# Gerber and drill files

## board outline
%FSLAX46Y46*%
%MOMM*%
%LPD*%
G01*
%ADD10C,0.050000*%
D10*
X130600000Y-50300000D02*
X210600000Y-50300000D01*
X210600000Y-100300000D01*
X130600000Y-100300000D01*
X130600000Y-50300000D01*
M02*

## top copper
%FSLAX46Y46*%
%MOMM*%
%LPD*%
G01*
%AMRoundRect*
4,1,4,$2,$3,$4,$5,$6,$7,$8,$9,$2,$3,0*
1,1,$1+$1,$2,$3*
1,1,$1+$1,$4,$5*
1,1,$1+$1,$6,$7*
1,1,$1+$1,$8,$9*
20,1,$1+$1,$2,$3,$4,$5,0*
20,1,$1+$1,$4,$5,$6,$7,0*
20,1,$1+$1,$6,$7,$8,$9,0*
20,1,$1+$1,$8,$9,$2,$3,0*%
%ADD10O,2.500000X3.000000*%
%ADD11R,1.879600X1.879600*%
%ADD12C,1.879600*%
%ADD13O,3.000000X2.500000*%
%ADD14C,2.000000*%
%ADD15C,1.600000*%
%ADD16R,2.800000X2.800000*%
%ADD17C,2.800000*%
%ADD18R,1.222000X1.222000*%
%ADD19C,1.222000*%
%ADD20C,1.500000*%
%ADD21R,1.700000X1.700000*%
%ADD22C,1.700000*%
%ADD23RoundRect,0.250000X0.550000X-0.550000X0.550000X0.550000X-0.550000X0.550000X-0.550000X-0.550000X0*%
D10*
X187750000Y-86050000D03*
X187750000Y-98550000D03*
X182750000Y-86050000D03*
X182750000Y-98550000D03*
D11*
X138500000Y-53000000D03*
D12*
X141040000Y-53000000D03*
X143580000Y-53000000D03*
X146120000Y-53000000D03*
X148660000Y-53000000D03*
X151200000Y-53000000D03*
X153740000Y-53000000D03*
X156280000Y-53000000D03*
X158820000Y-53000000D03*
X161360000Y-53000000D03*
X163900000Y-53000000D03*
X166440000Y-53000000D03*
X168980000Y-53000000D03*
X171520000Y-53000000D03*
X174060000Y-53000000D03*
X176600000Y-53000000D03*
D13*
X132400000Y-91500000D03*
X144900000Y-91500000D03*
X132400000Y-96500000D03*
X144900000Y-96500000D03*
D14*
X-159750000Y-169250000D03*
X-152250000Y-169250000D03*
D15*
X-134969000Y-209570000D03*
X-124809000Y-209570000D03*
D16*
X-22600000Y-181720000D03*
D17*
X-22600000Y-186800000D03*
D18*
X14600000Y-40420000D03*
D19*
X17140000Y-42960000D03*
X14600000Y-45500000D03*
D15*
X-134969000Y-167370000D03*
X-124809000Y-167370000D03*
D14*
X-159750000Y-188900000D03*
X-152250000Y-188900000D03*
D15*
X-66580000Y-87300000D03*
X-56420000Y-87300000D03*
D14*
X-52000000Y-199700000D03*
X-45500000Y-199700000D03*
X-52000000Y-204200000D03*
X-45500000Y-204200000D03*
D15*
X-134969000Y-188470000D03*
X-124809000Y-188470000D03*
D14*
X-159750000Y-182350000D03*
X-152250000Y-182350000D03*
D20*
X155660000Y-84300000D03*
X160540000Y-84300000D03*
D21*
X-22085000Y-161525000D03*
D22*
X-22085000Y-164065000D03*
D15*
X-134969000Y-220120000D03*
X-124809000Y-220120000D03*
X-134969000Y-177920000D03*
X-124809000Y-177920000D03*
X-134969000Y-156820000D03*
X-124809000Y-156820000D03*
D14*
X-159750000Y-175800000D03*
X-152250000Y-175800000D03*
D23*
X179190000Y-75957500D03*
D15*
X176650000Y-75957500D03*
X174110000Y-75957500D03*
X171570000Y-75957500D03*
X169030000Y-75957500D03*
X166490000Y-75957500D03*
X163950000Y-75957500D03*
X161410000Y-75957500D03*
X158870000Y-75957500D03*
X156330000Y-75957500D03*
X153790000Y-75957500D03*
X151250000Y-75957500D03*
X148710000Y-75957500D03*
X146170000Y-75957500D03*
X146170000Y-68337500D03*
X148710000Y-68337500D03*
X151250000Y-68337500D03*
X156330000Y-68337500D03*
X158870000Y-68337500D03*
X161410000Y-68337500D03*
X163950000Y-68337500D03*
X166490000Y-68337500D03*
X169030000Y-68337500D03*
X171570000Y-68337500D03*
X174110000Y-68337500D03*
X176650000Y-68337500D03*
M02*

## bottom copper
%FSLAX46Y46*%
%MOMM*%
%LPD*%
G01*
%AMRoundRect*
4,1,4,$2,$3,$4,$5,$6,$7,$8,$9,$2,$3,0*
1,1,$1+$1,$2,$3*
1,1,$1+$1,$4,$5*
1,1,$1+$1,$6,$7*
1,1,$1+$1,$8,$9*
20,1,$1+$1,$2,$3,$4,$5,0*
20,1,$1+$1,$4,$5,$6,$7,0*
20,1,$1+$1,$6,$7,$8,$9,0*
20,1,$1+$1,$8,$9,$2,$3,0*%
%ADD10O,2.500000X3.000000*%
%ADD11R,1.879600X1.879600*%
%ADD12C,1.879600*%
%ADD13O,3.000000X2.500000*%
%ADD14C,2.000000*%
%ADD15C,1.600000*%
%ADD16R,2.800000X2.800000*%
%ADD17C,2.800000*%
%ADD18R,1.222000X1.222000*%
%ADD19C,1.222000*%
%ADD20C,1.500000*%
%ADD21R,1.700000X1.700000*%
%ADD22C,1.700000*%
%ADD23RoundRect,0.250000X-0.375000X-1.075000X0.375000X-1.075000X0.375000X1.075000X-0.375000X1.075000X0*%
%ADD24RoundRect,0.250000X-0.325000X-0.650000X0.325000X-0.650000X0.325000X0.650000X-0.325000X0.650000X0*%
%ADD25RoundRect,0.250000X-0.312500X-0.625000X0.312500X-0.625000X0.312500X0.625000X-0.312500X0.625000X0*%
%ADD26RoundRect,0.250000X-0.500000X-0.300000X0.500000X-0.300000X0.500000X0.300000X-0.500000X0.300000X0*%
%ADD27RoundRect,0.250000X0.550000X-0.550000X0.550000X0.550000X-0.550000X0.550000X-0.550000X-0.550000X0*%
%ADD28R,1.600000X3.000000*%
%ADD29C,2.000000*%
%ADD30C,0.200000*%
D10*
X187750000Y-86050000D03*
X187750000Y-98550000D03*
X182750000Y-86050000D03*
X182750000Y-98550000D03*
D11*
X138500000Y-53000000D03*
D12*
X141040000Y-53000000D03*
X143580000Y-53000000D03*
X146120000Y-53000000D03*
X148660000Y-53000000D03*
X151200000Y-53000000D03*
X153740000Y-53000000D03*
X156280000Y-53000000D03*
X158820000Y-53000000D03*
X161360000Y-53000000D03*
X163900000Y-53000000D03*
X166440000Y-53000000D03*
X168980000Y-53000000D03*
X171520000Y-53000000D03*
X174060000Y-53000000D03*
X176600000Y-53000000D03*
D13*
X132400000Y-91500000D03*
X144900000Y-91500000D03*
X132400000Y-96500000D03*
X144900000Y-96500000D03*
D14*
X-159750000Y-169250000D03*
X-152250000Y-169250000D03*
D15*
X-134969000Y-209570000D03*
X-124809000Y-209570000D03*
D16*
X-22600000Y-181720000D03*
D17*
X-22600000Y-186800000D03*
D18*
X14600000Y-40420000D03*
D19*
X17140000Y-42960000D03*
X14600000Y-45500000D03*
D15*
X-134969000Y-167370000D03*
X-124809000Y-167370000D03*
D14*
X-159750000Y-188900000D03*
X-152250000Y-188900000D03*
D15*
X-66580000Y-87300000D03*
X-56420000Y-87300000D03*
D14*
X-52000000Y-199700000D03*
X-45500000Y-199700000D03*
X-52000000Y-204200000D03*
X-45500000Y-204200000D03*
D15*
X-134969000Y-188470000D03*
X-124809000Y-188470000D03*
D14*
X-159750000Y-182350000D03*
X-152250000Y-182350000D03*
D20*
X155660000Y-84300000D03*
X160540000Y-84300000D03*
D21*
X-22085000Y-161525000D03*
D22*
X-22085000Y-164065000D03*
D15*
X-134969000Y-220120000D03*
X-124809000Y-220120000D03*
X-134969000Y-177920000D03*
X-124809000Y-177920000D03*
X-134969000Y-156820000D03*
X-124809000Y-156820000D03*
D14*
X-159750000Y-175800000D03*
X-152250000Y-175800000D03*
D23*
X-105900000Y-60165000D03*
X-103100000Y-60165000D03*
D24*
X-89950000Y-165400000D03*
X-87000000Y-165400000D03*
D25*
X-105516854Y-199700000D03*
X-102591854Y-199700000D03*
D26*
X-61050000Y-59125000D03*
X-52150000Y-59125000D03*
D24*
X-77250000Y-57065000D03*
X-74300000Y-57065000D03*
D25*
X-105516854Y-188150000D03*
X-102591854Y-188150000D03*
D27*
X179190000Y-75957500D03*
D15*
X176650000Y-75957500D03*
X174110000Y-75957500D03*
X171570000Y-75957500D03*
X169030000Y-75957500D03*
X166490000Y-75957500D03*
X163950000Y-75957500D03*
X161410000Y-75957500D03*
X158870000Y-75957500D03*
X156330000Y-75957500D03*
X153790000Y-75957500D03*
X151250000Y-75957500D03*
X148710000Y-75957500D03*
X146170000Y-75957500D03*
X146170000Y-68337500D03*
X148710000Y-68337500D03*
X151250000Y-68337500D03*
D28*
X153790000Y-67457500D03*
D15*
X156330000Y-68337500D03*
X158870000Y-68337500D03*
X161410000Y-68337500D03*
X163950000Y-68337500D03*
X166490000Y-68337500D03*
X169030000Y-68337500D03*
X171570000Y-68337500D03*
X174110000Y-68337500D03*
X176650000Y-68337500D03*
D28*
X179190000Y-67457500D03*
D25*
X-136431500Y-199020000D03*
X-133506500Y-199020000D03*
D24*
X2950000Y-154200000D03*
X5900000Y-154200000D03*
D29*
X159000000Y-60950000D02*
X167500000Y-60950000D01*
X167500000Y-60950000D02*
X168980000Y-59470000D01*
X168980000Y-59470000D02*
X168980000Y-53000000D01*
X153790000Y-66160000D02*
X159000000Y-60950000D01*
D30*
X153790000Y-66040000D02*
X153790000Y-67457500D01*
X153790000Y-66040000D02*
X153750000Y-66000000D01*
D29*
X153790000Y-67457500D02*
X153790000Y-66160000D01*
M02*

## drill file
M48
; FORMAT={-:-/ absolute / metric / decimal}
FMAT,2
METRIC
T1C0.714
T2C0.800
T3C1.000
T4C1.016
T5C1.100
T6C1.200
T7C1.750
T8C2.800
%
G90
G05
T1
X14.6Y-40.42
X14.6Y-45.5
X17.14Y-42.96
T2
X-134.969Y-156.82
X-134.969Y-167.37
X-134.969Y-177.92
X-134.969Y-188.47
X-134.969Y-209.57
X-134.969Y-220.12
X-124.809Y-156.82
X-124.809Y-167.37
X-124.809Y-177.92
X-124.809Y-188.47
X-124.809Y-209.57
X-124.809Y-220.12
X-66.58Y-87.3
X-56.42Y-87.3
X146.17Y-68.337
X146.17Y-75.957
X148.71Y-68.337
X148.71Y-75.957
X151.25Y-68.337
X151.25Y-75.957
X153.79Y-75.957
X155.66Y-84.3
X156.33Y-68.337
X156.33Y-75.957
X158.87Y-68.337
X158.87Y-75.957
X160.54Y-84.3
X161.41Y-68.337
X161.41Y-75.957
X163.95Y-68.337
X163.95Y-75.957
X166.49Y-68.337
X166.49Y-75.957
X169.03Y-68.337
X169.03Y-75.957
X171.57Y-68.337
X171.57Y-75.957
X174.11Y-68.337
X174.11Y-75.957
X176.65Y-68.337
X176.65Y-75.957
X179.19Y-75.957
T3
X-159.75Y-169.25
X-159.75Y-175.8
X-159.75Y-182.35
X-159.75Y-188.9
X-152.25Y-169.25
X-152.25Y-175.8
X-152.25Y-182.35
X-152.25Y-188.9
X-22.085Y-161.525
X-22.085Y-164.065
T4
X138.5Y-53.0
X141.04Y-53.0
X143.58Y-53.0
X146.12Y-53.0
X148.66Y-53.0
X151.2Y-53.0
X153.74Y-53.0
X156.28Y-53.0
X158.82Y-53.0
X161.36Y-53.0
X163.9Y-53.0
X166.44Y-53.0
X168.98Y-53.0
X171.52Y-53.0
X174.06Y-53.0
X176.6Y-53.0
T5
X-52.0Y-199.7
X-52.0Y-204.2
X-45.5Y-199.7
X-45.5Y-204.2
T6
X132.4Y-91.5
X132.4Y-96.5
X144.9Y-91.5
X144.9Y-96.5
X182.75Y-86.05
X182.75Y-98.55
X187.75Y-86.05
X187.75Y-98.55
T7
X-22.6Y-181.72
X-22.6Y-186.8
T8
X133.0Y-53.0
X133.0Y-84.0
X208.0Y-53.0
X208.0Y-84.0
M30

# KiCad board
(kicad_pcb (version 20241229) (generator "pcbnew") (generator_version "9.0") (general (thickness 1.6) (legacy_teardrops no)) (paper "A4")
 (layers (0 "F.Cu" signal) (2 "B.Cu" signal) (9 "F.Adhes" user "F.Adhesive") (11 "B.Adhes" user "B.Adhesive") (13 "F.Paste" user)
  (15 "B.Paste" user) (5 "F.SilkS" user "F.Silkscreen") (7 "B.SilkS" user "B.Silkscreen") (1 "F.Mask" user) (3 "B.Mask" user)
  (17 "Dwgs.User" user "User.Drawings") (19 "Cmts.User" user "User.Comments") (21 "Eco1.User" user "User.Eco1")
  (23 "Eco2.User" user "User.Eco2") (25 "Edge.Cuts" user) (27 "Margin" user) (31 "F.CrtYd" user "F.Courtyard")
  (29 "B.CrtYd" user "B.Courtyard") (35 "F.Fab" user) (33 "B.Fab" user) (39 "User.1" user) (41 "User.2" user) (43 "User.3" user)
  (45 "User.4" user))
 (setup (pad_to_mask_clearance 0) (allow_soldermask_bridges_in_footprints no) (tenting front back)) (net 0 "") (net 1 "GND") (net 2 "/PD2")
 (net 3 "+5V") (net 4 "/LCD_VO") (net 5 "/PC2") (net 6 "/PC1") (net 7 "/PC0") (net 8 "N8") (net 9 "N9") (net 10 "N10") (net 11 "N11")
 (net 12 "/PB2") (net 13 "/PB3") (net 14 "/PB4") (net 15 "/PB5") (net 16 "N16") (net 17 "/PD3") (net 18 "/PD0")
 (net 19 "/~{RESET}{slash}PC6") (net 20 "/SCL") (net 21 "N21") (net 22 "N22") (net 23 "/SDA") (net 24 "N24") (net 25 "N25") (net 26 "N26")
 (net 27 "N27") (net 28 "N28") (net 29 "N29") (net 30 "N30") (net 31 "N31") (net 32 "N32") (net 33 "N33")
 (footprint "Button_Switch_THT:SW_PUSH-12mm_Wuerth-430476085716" (layer "F.Cu") (at 187.75 86.05 -90)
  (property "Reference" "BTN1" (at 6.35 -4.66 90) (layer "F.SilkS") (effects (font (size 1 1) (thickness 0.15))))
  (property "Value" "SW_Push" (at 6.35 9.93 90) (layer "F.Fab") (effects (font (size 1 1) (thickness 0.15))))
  (pad "1" thru_hole oval (at 0 0 270) (size 3 2.5) (drill 1.2) (layers "*.Cu" "*.Mask") (remove_unused_layers no) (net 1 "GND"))
  (pad "1" thru_hole oval (at 12.5 0 270) (size 3 2.5) (drill 1.2) (layers "*.Cu" "*.Mask") (remove_unused_layers no) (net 1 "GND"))
  (pad "2" thru_hole oval (at 0 5 270) (size 3 2.5) (drill 1.2) (layers "*.Cu" "*.Mask") (remove_unused_layers no) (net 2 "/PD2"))
  (pad "2" thru_hole oval (at 12.5 5 270) (size 3 2.5) (drill 1.2) (layers "*.Cu" "*.Mask") (remove_unused_layers no) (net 2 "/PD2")))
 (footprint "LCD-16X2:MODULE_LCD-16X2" (layer "F.Cu") (at 170.5 68.5)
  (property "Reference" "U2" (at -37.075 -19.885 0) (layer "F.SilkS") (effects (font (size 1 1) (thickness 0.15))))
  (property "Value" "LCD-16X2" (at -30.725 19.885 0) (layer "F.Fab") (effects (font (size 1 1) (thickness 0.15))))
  (pad "" np_thru_hole circle (at -37.5 -15.5) (size 2.8 2.8) (drill 2.8) (layers "*.Cu" "*.Mask"))
  (pad "" np_thru_hole circle (at -37.5 15.5) (size 2.8 2.8) (drill 2.8) (layers "*.Cu" "*.Mask"))
  (pad "" np_thru_hole circle (at 37.5 -15.5) (size 2.8 2.8) (drill 2.8) (layers "*.Cu" "*.Mask"))
  (pad "" np_thru_hole circle (at 37.5 15.5) (size 2.8 2.8) (drill 2.8) (layers "*.Cu" "*.Mask"))
  (pad "1" thru_hole rect (at -32 -15.5) (size 1.8796 1.8796) (drill 1.016) (layers "*.Cu" "*.Mask") (remove_unused_layers no) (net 1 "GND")
   (solder_mask_margin 0.102))
  (pad "2" thru_hole circle (at -29.46 -15.5) (size 1.8796 1.8796) (drill 1.016) (layers "*.Cu" "*.Mask") (remove_unused_layers no)
   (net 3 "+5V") (solder_mask_margin 0.102))
  (pad "3" thru_hole circle (at -26.92 -15.5) (size 1.8796 1.8796) (drill 1.016) (layers "*.Cu" "*.Mask") (remove_unused_layers no)
   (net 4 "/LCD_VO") (solder_mask_margin 0.102))
  (pad "4" thru_hole circle (at -24.38 -15.5) (size 1.8796 1.8796) (drill 1.016) (layers "*.Cu" "*.Mask") (remove_unused_layers no)
   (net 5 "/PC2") (solder_mask_margin 0.102))
  (pad "5" thru_hole circle (at -21.84 -15.5) (size 1.8796 1.8796) (drill 1.016) (layers "*.Cu" "*.Mask") (remove_unused_layers no)
   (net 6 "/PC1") (solder_mask_margin 0.102))
  (pad "6" thru_hole circle (at -19.3 -15.5) (size 1.8796 1.8796) (drill 1.016) (layers "*.Cu" "*.Mask") (remove_unused_layers no)
   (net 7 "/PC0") (solder_mask_margin 0.102))
  (pad "7" thru_hole circle (at -16.76 -15.5) (size 1.8796 1.8796) (drill 1.016) (layers "*.Cu" "*.Mask") (remove_unused_layers no)
   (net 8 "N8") (solder_mask_margin 0.102))
  (pad "8" thru_hole circle (at -14.22 -15.5) (size 1.8796 1.8796) (drill 1.016) (layers "*.Cu" "*.Mask") (remove_unused_layers no)
   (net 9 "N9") (solder_mask_margin 0.102))
  (pad "9" thru_hole circle (at -11.68 -15.5) (size 1.8796 1.8796) (drill 1.016) (layers "*.Cu" "*.Mask") (remove_unused_layers no)
   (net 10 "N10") (solder_mask_margin 0.102))
  (pad "10" thru_hole circle (at -9.14 -15.5) (size 1.8796 1.8796) (drill 1.016) (layers "*.Cu" "*.Mask") (remove_unused_layers no)
   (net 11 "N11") (solder_mask_margin 0.102))
  (pad "11" thru_hole circle (at -6.6 -15.5) (size 1.8796 1.8796) (drill 1.016) (layers "*.Cu" "*.Mask") (remove_unused_layers no)
   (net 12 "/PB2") (solder_mask_margin 0.102))
  (pad "12" thru_hole circle (at -4.06 -15.5) (size 1.8796 1.8796) (drill 1.016) (layers "*.Cu" "*.Mask") (remove_unused_layers no)
   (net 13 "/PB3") (solder_mask_margin 0.102))
  (pad "13" thru_hole circle (at -1.52 -15.5) (size 1.8796 1.8796) (drill 1.016) (layers "*.Cu" "*.Mask") (remove_unused_layers no)
   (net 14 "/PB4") (solder_mask_margin 0.102))
  (pad "14" thru_hole circle (at 1.02 -15.5) (size 1.8796 1.8796) (drill 1.016) (layers "*.Cu" "*.Mask") (remove_unused_layers no)
   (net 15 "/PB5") (solder_mask_margin 0.102))
  (pad "15" thru_hole circle (at 3.56 -15.5) (size 1.8796 1.8796) (drill 1.016) (layers "*.Cu" "*.Mask") (remove_unused_layers no)
   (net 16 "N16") (solder_mask_margin 0.102))
  (pad "16" thru_hole circle (at 6.1 -15.5) (size 1.8796 1.8796) (drill 1.016) (layers "*.Cu" "*.Mask") (remove_unused_layers no)
   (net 1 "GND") (solder_mask_margin 0.102)))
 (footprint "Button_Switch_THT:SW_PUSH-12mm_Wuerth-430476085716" (layer "F.Cu") (at 132.4 91.5)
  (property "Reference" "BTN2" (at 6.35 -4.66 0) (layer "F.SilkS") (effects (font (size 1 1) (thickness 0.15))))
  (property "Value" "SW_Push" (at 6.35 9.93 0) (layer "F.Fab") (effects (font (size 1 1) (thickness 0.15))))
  (pad "1" thru_hole oval (at 0 0) (size 3 2.5) (drill 1.2) (layers "*.Cu" "*.Mask") (remove_unused_layers no) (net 1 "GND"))
  (pad "1" thru_hole oval (at 12.5 0) (size 3 2.5) (drill 1.2) (layers "*.Cu" "*.Mask") (remove_unused_layers no) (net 1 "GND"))
  (pad "2" thru_hole oval (at 0 5) (size 3 2.5) (drill 1.2) (layers "*.Cu" "*.Mask") (remove_unused_layers no) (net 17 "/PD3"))
  (pad "2" thru_hole oval (at 12.5 5) (size 3 2.5) (drill 1.2) (layers "*.Cu" "*.Mask") (remove_unused_layers no) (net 17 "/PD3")))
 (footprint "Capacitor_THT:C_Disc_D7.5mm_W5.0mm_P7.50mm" (layer "F.Cu") (at -159.75 169.25)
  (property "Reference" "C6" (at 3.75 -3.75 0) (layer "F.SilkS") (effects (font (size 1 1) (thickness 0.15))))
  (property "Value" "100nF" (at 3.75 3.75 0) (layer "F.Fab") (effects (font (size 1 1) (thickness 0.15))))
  (pad "1" thru_hole circle (at 0 0) (size 2 2) (drill 1) (layers "*.Cu" "*.Mask") (remove_unused_layers no) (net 1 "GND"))
  (pad "2" thru_hole circle (at 7.5 0) (size 2 2) (drill 1) (layers "*.Cu" "*.Mask") (remove_unused_layers no) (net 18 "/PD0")))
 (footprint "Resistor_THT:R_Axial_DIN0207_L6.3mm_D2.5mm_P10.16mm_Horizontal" (layer "F.Cu") (at -134.969 209.57)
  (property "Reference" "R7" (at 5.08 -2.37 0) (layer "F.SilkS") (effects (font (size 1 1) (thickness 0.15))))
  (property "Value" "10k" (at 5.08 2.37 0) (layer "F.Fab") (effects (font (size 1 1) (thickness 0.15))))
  (pad "1" thru_hole circle (at 0 0) (size 1.6 1.6) (drill 0.8) (layers "*.Cu" "*.Mask") (remove_unused_layers no) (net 3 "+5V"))
  (pad "2" thru_hole circle (at 10.16 0) (size 1.6 1.6) (drill 0.8) (layers "*.Cu" "*.Mask") (remove_unused_layers no)
   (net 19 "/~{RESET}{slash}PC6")))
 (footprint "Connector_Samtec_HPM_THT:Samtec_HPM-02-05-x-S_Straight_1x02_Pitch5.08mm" (layer "F.Cu") (at -22.6 181.72)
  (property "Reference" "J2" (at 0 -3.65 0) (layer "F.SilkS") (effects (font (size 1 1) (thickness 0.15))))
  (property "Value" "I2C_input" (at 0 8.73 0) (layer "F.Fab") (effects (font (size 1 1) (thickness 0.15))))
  (pad "1" thru_hole rect (at 0 0) (size 2.8 2.8) (drill 1.75) (layers "*.Cu" "*.Mask") (remove_unused_layers no) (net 3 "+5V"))
  (pad "2" thru_hole circle (at 0 5.08) (size 2.8 2.8) (drill 1.75) (layers "*.Cu" "*.Mask") (remove_unused_layers no) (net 1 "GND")))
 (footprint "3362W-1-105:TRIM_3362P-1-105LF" (layer "F.Cu") (at 14.6 42.96 -90)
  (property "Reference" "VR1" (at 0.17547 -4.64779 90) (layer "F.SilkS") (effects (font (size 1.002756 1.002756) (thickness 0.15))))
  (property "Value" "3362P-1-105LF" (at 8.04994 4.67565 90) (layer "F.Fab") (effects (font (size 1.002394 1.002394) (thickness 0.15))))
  (pad "1" thru_hole rect (at -2.54 0 270) (size 1.222 1.222) (drill 0.714) (layers "*.Cu" "*.Mask") (remove_unused_layers no) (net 3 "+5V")
   (solder_mask_margin 0.102))
  (pad "2" thru_hole circle (at 0 -2.54 270) (size 1.222 1.222) (drill 0.714) (layers "*.Cu" "*.Mask") (remove_unused_layers no)
   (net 4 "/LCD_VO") (solder_mask_margin 0.102))
  (pad "3" thru_hole circle (at 2.54 0 270) (size 1.222 1.222) (drill 0.714) (layers "*.Cu" "*.Mask") (remove_unused_layers no)
   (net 1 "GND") (solder_mask_margin 0.102)))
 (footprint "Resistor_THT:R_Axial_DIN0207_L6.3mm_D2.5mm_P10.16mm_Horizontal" (layer "F.Cu") (at -134.969 167.37)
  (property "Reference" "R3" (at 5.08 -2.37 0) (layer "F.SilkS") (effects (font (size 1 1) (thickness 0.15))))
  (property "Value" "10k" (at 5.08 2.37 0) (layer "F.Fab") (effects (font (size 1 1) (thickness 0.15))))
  (pad "1" thru_hole circle (at 0 0) (size 1.6 1.6) (drill 0.8) (layers "*.Cu" "*.Mask") (remove_unused_layers no) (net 3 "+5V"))
  (pad "2" thru_hole circle (at 10.16 0) (size 1.6 1.6) (drill 0.8) (layers "*.Cu" "*.Mask") (remove_unused_layers no) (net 17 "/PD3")))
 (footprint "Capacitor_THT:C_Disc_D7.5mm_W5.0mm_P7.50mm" (layer "F.Cu") (at -159.75 188.9)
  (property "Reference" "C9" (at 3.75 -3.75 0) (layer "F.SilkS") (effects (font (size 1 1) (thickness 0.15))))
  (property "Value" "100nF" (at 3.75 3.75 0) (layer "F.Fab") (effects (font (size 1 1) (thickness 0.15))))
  (pad "1" thru_hole circle (at 0 0) (size 2 2) (drill 1) (layers "*.Cu" "*.Mask") (remove_unused_layers no) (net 1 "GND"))
  (pad "2" thru_hole circle (at 7.5 0) (size 2 2) (drill 1) (layers "*.Cu" "*.Mask") (remove_unused_layers no) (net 17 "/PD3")))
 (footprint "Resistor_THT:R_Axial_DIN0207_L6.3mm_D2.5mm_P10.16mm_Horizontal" (layer "F.Cu") (at -66.58 87.3)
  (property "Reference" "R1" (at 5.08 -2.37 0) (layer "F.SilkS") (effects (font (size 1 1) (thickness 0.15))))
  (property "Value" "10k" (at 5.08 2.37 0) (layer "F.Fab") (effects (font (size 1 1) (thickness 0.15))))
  (pad "1" thru_hole circle (at 0 0) (size 1.6 1.6) (drill 0.8) (layers "*.Cu" "*.Mask") (remove_unused_layers no) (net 3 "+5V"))
  (pad "2" thru_hole circle (at 10.16 0) (size 1.6 1.6) (drill 0.8) (layers "*.Cu" "*.Mask") (remove_unused_layers no) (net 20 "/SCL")))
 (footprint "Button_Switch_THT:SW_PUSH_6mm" (layer "F.Cu") (at -52 199.7)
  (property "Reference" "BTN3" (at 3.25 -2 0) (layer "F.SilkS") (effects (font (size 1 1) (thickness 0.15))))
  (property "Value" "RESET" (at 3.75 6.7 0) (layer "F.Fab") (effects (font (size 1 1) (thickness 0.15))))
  (pad "1" thru_hole circle (at 0 0 90) (size 2 2) (drill 1.1) (layers "*.Cu" "*.Mask") (remove_unused_layers no) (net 1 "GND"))
  (pad "1" thru_hole circle (at 6.5 0 90) (size 2 2) (drill 1.1) (layers "*.Cu" "*.Mask") (remove_unused_layers no) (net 1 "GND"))
  (pad "2" thru_hole circle (at 0 4.5 90) (size 2 2) (drill 1.1) (layers "*.Cu" "*.Mask") (remove_unused_layers no)
   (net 19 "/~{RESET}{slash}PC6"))
  (pad "2" thru_hole circle (at 6.5 4.5 90) (size 2 2) (drill 1.1) (layers "*.Cu" "*.Mask") (remove_unused_layers no)
   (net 19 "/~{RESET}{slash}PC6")))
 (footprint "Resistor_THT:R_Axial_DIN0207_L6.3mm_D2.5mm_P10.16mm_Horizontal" (layer "F.Cu") (at -134.969 188.47)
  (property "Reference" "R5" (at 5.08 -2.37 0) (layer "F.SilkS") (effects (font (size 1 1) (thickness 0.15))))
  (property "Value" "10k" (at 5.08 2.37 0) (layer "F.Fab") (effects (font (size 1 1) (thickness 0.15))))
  (pad "1" thru_hole circle (at 0 0) (size 1.6 1.6) (drill 0.8) (layers "*.Cu" "*.Mask") (remove_unused_layers no) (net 3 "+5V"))
  (pad "2" thru_hole circle (at 10.16 0) (size 1.6 1.6) (drill 0.8) (layers "*.Cu" "*.Mask") (remove_unused_layers no) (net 18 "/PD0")))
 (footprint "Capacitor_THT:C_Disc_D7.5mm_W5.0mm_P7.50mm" (layer "F.Cu") (at -159.75 182.35)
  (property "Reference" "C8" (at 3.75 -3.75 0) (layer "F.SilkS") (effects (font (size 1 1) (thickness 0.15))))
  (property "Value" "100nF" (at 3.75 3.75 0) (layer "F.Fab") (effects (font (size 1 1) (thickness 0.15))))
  (pad "1" thru_hole circle (at 0 0) (size 2 2) (drill 1) (layers "*.Cu" "*.Mask") (remove_unused_layers no) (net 1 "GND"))
  (pad "2" thru_hole circle (at 7.5 0) (size 2 2) (drill 1) (layers "*.Cu" "*.Mask") (remove_unused_layers no) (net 2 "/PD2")))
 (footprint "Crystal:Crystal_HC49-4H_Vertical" (layer "F.Cu") (at 155.66 84.3)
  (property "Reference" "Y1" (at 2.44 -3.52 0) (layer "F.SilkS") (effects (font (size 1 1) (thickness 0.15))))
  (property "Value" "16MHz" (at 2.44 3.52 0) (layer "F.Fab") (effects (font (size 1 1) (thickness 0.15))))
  (pad "1" thru_hole circle (at 0 0) (size 1.5 1.5) (drill 0.8) (layers "*.Cu" "*.Mask") (remove_unused_layers no) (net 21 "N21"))
  (pad "2" thru_hole circle (at 4.88 0) (size 1.5 1.5) (drill 0.8) (layers "*.Cu" "*.Mask") (remove_unused_layers no) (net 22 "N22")))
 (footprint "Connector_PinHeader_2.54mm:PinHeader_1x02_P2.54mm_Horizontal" (layer "F.Cu") (at -22.085 161.525)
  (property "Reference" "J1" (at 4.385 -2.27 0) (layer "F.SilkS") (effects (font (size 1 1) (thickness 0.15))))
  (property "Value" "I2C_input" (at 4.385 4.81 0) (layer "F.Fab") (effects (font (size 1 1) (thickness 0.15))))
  (pad "1" thru_hole rect (at 0 0) (size 1.7 1.7) (drill 1) (layers "*.Cu" "*.Mask") (remove_unused_layers no) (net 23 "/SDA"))
  (pad "2" thru_hole circle (at 0 2.54) (size 1.7 1.7) (drill 1) (layers "*.Cu" "*.Mask") (remove_unused_layers no) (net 20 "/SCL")))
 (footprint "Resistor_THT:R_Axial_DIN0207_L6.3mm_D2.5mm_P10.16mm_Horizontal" (layer "F.Cu") (at -134.969 220.12)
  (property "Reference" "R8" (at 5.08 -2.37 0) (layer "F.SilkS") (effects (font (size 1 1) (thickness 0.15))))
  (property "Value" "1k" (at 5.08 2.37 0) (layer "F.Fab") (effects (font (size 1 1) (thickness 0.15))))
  (pad "1" thru_hole circle (at 0 0) (size 1.6 1.6) (drill 0.8) (layers "*.Cu" "*.Mask") (remove_unused_layers no) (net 3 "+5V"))
  (pad "2" thru_hole circle (at 10.16 0) (size 1.6 1.6) (drill 0.8) (layers "*.Cu" "*.Mask") (remove_unused_layers no) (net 16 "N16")))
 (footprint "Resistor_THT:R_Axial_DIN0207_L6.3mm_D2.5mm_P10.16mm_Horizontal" (layer "F.Cu") (at -134.969 177.92)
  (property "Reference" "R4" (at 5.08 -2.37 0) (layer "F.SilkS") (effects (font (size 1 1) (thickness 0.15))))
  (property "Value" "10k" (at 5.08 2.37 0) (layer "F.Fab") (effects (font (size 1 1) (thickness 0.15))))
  (pad "1" thru_hole circle (at 0 0) (size 1.6 1.6) (drill 0.8) (layers "*.Cu" "*.Mask") (remove_unused_layers no) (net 3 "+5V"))
  (pad "2" thru_hole circle (at 10.16 0) (size 1.6 1.6) (drill 0.8) (layers "*.Cu" "*.Mask") (remove_unused_layers no) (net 2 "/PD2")))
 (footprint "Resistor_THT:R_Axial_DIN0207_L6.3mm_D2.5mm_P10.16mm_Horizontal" (layer "F.Cu") (at -134.969 156.82)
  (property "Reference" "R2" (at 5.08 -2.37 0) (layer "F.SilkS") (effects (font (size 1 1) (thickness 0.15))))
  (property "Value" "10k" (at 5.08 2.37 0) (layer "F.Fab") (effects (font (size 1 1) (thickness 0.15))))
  (pad "1" thru_hole circle (at 0 0) (size 1.6 1.6) (drill 0.8) (layers "*.Cu" "*.Mask") (remove_unused_layers no) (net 3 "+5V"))
  (pad "2" thru_hole circle (at 10.16 0) (size 1.6 1.6) (drill 0.8) (layers "*.Cu" "*.Mask") (remove_unused_layers no) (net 23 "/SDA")))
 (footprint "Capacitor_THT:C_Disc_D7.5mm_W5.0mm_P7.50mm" (layer "F.Cu") (at -159.75 175.8)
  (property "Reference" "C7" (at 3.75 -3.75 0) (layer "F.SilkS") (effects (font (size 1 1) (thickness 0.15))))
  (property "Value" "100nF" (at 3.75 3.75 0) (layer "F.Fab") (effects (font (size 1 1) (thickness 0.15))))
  (pad "1" thru_hole circle (at 0 0) (size 2 2) (drill 1) (layers "*.Cu" "*.Mask") (remove_unused_layers no) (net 1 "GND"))
  (pad "2" thru_hole circle (at 7.5 0) (size 2 2) (drill 1) (layers "*.Cu" "*.Mask") (remove_unused_layers no)
   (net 19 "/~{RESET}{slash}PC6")))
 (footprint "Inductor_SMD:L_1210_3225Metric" (layer "B.Cu") (at -104.5 60.165)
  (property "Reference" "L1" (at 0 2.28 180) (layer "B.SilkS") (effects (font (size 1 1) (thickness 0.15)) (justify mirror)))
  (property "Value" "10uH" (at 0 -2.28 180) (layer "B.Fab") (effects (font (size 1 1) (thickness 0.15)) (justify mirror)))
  (pad "1" smd roundrect (at -1.4 0) (size 1.25 2.65) (layers "B.Cu" "B.Mask" "B.Paste") (roundrect_rratio 0.2) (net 3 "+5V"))
  (pad "2" smd roundrect (at 1.4 0) (size 1.25 2.65) (layers "B.Cu" "B.Mask" "B.Paste") (roundrect_rratio 0.2) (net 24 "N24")))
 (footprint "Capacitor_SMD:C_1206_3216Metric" (layer "B.Cu") (at -88.475 165.4)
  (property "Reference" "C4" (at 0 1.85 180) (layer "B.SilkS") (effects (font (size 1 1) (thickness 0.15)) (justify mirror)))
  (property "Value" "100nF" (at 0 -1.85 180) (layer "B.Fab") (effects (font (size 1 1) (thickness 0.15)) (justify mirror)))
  (pad "1" smd roundrect (at -1.475 0) (size 1.15 1.8) (layers "B.Cu" "B.Mask" "B.Paste") (roundrect_rratio 0.217391) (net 1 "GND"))
  (pad "2" smd roundrect (at 1.475 0) (size 1.15 1.8) (layers "B.Cu" "B.Mask" "B.Paste") (roundrect_rratio 0.217391) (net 24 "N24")))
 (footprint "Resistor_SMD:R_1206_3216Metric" (layer "B.Cu") (at -104.054354 199.7)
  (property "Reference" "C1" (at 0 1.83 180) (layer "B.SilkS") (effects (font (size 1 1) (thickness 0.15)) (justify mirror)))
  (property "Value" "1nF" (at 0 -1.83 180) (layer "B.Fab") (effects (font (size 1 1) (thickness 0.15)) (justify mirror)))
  (pad "1" smd roundrect (at -1.4625 0) (size 1.125 1.75) (layers "B.Cu" "B.Mask" "B.Paste") (roundrect_rratio 0.222222) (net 22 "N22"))
  (pad "2" smd roundrect (at 1.4625 0) (size 1.125 1.75) (layers "B.Cu" "B.Mask" "B.Paste") (roundrect_rratio 0.222222) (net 1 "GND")))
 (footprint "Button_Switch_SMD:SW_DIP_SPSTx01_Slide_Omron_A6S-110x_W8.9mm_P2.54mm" (layer "B.Cu") (at -56.6 59.125)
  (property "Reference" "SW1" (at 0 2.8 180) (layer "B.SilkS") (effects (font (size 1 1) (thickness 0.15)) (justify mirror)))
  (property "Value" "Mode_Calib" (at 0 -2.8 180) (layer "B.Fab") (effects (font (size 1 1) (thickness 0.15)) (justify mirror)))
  (pad "1" smd roundrect (at -4.45 0) (size 1.5 1.1) (layers "B.Cu" "B.Mask" "B.Paste") (roundrect_rratio 0.227273) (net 1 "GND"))
  (pad "2" smd roundrect (at 4.45 0) (size 1.5 1.1) (layers "B.Cu" "B.Mask" "B.Paste") (roundrect_rratio 0.227273) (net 18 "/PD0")))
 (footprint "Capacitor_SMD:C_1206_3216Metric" (layer "B.Cu") (at -75.775 57.065)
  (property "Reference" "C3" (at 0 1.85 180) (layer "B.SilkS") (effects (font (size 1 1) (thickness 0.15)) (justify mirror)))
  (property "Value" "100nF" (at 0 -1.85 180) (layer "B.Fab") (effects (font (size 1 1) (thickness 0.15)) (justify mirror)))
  (pad "1" smd roundrect (at -1.475 0) (size 1.15 1.8) (layers "B.Cu" "B.Mask" "B.Paste") (roundrect_rratio 0.217391) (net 1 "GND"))
  (pad "2" smd roundrect (at 1.475 0) (size 1.15 1.8) (layers "B.Cu" "B.Mask" "B.Paste") (roundrect_rratio 0.217391) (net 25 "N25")))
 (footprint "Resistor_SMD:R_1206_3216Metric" (layer "B.Cu") (at -104.054354 188.15)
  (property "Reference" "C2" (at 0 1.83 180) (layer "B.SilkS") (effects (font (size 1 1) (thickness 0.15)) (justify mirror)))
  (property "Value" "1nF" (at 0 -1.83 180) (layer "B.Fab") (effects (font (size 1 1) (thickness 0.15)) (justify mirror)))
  (pad "1" smd roundrect (at -1.4625 0) (size 1.125 1.75) (layers "B.Cu" "B.Mask" "B.Paste") (roundrect_rratio 0.222222) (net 1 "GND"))
  (pad "2" smd roundrect (at 1.4625 0) (size 1.125 1.75) (layers "B.Cu" "B.Mask" "B.Paste") (roundrect_rratio 0.222222) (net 21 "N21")))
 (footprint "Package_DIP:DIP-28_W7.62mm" (layer "B.Cu") (at 179.19 75.9575 90)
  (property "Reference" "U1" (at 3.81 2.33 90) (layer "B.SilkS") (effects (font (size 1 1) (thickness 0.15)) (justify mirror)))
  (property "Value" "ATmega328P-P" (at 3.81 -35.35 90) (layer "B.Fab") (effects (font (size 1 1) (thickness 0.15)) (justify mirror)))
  (pad "1" thru_hole roundrect (at 0 0 90) (size 1.6 1.6) (drill 0.8) (layers "*.Cu" "*.Mask") (remove_unused_layers no)
   (roundrect_rratio 0.15625) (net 19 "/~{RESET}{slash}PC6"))
  (pad "2" thru_hole circle (at 0 -2.54 90) (size 1.6 1.6) (drill 0.8) (layers "*.Cu" "*.Mask") (remove_unused_layers no) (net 18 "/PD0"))
  (pad "3" thru_hole circle (at 0 -5.08 90) (size 1.6 1.6) (drill 0.8) (layers "*.Cu" "*.Mask") (remove_unused_layers no) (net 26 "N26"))
  (pad "4" thru_hole circle (at 0 -7.62 90) (size 1.6 1.6) (drill 0.8) (layers "*.Cu" "*.Mask") (remove_unused_layers no) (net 2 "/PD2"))
  (pad "5" thru_hole circle (at 0 -10.16 90) (size 1.6 1.6) (drill 0.8) (layers "*.Cu" "*.Mask") (remove_unused_layers no) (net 17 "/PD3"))
  (pad "6" thru_hole circle (at 0 -12.7 90) (size 1.6 1.6) (drill 0.8) (layers "*.Cu" "*.Mask") (remove_unused_layers no) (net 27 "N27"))
  (pad "7" thru_hole circle (at 0 -15.24 90) (size 1.6 1.6) (drill 0.8) (layers "*.Cu" "*.Mask") (remove_unused_layers no) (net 3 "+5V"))
  (pad "8" thru_hole circle (at 0 -17.78 90) (size 1.6 1.6) (drill 0.8) (layers "*.Cu" "*.Mask") (remove_unused_layers no) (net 1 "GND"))
  (pad "9" thru_hole circle (at 0 -20.32 90) (size 1.6 1.6) (drill 0.8) (layers "*.Cu" "*.Mask") (remove_unused_layers no) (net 22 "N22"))
  (pad "10" thru_hole circle (at 0 -22.86 90) (size 1.6 1.6) (drill 0.8) (layers "*.Cu" "*.Mask") (remove_unused_layers no) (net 21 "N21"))
  (pad "11" thru_hole circle (at 0 -25.4 90) (size 1.6 1.6) (drill 0.8) (layers "*.Cu" "*.Mask") (remove_unused_layers no) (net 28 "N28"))
  (pad "12" thru_hole circle (at 0 -27.94 90) (size 1.6 1.6) (drill 0.8) (layers "*.Cu" "*.Mask") (remove_unused_layers no) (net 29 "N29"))
  (pad "13" thru_hole circle (at 0 -30.48 90) (size 1.6 1.6) (drill 0.8) (layers "*.Cu" "*.Mask") (remove_unused_layers no) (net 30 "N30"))
  (pad "14" thru_hole circle (at 0 -33.02 90) (size 1.6 1.6) (drill 0.8) (layers "*.Cu" "*.Mask") (remove_unused_layers no) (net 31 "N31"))
  (pad "15" thru_hole circle (at 7.62 -33.02 90) (size 1.6 1.6) (drill 0.8) (layers "*.Cu" "*.Mask") (remove_unused_layers no)
   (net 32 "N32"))
  (pad "16" thru_hole circle (at 7.62 -30.48 90) (size 1.6 1.6) (drill 0.8) (layers "*.Cu" "*.Mask") (remove_unused_layers no)
   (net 12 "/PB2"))
  (pad "17" thru_hole circle (at 7.62 -27.94 90) (size 1.6 1.6) (drill 0.8) (layers "*.Cu" "*.Mask") (remove_unused_layers no)
   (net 13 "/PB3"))
  (pad "18" smd rect (at 8.5 -25.4 90) (size 3 1.6) (layers "B.Cu" "B.Mask" "B.Paste") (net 14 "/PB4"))
  (pad "19" thru_hole circle (at 7.62 -22.86 90) (size 1.6 1.6) (drill 0.8) (layers "*.Cu" "*.Mask") (remove_unused_layers no)
   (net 15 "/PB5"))
  (pad "20" thru_hole circle (at 7.62 -20.32 90) (size 1.6 1.6) (drill 0.8) (layers "*.Cu" "*.Mask") (remove_unused_layers no)
   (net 24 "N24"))
  (pad "21" thru_hole circle (at 7.62 -17.78 90) (size 1.6 1.6) (drill 0.8) (layers "*.Cu" "*.Mask") (remove_unused_layers no)
   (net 25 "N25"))
  (pad "22" thru_hole circle (at 7.62 -15.24 90) (size 1.6 1.6) (drill 0.8) (layers "*.Cu" "*.Mask") (remove_unused_layers no) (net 1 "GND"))
  (pad "23" thru_hole circle (at 7.62 -12.7 90) (size 1.6 1.6) (drill 0.8) (layers "*.Cu" "*.Mask") (remove_unused_layers no) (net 7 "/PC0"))
  (pad "24" thru_hole circle (at 7.62 -10.16 90) (size 1.6 1.6) (drill 0.8) (layers "*.Cu" "*.Mask") (remove_unused_layers no)
   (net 6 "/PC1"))
  (pad "25" thru_hole circle (at 7.62 -7.62 90) (size 1.6 1.6) (drill 0.8) (layers "*.Cu" "*.Mask") (remove_unused_layers no) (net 5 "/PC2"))
  (pad "26" thru_hole circle (at 7.62 -5.08 90) (size 1.6 1.6) (drill 0.8) (layers "*.Cu" "*.Mask") (remove_unused_layers no) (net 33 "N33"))
  (pad "27" thru_hole circle (at 7.62 -2.54 90) (size 1.6 1.6) (drill 0.8) (layers "*.Cu" "*.Mask") (remove_unused_layers no)
   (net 23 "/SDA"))
  (pad "28" smd rect (at 8.5 0 90) (size 3 1.6) (layers "B.Cu" "B.Mask" "B.Paste") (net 20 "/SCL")))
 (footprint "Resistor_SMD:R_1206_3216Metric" (layer "B.Cu") (at -134.969 199.02)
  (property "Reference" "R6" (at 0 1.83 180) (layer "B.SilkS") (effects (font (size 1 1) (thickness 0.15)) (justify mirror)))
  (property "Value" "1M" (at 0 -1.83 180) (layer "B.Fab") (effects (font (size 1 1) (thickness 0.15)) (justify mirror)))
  (pad "1" smd roundrect (at -1.4625 0) (size 1.125 1.75) (layers "B.Cu" "B.Mask" "B.Paste") (roundrect_rratio 0.222222) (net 22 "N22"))
  (pad "2" smd roundrect (at 1.4625 0) (size 1.125 1.75) (layers "B.Cu" "B.Mask" "B.Paste") (roundrect_rratio 0.222222) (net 21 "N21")))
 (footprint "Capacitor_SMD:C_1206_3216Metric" (layer "B.Cu") (at 4.425 154.2)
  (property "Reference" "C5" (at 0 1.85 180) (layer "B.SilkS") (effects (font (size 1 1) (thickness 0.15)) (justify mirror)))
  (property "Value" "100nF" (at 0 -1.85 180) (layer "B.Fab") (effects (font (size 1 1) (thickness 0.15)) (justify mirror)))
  (pad "1" smd roundrect (at -1.475 0) (size 1.15 1.8) (layers "B.Cu" "B.Mask" "B.Paste") (roundrect_rratio 0.217391) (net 1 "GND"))
  (pad "2" smd roundrect (at 1.475 0) (size 1.15 1.8) (layers "B.Cu" "B.Mask" "B.Paste") (roundrect_rratio 0.217391) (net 3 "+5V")))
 (gr_rect (start 130.6 50.3) (end 210.6 100.3) (stroke (width 0.05) (type solid)) (fill no) (layer "Edge.Cuts"))
 (segment (start 159 60.95) (end 167.5 60.95) (width 2) (layer "B.Cu") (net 14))
 (segment (start 167.5 60.95) (end 168.98 59.47) (width 2) (layer "B.Cu") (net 14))
 (segment (start 168.98 59.47) (end 168.98 53) (width 2) (layer "B.Cu") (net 14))
 (segment (start 153.79 66.16) (end 159 60.95) (width 2) (layer "B.Cu") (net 14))
 (segment (start 153.79 66.04) (end 153.79 67.4575) (width 0.2) (layer "B.Cu") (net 14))
 (segment (start 153.79 66.04) (end 153.75 66) (width 0.2) (layer "B.Cu") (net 14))
 (segment (start 153.79 67.4575) (end 153.79 66.16) (width 2) (layer "B.Cu") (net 14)))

